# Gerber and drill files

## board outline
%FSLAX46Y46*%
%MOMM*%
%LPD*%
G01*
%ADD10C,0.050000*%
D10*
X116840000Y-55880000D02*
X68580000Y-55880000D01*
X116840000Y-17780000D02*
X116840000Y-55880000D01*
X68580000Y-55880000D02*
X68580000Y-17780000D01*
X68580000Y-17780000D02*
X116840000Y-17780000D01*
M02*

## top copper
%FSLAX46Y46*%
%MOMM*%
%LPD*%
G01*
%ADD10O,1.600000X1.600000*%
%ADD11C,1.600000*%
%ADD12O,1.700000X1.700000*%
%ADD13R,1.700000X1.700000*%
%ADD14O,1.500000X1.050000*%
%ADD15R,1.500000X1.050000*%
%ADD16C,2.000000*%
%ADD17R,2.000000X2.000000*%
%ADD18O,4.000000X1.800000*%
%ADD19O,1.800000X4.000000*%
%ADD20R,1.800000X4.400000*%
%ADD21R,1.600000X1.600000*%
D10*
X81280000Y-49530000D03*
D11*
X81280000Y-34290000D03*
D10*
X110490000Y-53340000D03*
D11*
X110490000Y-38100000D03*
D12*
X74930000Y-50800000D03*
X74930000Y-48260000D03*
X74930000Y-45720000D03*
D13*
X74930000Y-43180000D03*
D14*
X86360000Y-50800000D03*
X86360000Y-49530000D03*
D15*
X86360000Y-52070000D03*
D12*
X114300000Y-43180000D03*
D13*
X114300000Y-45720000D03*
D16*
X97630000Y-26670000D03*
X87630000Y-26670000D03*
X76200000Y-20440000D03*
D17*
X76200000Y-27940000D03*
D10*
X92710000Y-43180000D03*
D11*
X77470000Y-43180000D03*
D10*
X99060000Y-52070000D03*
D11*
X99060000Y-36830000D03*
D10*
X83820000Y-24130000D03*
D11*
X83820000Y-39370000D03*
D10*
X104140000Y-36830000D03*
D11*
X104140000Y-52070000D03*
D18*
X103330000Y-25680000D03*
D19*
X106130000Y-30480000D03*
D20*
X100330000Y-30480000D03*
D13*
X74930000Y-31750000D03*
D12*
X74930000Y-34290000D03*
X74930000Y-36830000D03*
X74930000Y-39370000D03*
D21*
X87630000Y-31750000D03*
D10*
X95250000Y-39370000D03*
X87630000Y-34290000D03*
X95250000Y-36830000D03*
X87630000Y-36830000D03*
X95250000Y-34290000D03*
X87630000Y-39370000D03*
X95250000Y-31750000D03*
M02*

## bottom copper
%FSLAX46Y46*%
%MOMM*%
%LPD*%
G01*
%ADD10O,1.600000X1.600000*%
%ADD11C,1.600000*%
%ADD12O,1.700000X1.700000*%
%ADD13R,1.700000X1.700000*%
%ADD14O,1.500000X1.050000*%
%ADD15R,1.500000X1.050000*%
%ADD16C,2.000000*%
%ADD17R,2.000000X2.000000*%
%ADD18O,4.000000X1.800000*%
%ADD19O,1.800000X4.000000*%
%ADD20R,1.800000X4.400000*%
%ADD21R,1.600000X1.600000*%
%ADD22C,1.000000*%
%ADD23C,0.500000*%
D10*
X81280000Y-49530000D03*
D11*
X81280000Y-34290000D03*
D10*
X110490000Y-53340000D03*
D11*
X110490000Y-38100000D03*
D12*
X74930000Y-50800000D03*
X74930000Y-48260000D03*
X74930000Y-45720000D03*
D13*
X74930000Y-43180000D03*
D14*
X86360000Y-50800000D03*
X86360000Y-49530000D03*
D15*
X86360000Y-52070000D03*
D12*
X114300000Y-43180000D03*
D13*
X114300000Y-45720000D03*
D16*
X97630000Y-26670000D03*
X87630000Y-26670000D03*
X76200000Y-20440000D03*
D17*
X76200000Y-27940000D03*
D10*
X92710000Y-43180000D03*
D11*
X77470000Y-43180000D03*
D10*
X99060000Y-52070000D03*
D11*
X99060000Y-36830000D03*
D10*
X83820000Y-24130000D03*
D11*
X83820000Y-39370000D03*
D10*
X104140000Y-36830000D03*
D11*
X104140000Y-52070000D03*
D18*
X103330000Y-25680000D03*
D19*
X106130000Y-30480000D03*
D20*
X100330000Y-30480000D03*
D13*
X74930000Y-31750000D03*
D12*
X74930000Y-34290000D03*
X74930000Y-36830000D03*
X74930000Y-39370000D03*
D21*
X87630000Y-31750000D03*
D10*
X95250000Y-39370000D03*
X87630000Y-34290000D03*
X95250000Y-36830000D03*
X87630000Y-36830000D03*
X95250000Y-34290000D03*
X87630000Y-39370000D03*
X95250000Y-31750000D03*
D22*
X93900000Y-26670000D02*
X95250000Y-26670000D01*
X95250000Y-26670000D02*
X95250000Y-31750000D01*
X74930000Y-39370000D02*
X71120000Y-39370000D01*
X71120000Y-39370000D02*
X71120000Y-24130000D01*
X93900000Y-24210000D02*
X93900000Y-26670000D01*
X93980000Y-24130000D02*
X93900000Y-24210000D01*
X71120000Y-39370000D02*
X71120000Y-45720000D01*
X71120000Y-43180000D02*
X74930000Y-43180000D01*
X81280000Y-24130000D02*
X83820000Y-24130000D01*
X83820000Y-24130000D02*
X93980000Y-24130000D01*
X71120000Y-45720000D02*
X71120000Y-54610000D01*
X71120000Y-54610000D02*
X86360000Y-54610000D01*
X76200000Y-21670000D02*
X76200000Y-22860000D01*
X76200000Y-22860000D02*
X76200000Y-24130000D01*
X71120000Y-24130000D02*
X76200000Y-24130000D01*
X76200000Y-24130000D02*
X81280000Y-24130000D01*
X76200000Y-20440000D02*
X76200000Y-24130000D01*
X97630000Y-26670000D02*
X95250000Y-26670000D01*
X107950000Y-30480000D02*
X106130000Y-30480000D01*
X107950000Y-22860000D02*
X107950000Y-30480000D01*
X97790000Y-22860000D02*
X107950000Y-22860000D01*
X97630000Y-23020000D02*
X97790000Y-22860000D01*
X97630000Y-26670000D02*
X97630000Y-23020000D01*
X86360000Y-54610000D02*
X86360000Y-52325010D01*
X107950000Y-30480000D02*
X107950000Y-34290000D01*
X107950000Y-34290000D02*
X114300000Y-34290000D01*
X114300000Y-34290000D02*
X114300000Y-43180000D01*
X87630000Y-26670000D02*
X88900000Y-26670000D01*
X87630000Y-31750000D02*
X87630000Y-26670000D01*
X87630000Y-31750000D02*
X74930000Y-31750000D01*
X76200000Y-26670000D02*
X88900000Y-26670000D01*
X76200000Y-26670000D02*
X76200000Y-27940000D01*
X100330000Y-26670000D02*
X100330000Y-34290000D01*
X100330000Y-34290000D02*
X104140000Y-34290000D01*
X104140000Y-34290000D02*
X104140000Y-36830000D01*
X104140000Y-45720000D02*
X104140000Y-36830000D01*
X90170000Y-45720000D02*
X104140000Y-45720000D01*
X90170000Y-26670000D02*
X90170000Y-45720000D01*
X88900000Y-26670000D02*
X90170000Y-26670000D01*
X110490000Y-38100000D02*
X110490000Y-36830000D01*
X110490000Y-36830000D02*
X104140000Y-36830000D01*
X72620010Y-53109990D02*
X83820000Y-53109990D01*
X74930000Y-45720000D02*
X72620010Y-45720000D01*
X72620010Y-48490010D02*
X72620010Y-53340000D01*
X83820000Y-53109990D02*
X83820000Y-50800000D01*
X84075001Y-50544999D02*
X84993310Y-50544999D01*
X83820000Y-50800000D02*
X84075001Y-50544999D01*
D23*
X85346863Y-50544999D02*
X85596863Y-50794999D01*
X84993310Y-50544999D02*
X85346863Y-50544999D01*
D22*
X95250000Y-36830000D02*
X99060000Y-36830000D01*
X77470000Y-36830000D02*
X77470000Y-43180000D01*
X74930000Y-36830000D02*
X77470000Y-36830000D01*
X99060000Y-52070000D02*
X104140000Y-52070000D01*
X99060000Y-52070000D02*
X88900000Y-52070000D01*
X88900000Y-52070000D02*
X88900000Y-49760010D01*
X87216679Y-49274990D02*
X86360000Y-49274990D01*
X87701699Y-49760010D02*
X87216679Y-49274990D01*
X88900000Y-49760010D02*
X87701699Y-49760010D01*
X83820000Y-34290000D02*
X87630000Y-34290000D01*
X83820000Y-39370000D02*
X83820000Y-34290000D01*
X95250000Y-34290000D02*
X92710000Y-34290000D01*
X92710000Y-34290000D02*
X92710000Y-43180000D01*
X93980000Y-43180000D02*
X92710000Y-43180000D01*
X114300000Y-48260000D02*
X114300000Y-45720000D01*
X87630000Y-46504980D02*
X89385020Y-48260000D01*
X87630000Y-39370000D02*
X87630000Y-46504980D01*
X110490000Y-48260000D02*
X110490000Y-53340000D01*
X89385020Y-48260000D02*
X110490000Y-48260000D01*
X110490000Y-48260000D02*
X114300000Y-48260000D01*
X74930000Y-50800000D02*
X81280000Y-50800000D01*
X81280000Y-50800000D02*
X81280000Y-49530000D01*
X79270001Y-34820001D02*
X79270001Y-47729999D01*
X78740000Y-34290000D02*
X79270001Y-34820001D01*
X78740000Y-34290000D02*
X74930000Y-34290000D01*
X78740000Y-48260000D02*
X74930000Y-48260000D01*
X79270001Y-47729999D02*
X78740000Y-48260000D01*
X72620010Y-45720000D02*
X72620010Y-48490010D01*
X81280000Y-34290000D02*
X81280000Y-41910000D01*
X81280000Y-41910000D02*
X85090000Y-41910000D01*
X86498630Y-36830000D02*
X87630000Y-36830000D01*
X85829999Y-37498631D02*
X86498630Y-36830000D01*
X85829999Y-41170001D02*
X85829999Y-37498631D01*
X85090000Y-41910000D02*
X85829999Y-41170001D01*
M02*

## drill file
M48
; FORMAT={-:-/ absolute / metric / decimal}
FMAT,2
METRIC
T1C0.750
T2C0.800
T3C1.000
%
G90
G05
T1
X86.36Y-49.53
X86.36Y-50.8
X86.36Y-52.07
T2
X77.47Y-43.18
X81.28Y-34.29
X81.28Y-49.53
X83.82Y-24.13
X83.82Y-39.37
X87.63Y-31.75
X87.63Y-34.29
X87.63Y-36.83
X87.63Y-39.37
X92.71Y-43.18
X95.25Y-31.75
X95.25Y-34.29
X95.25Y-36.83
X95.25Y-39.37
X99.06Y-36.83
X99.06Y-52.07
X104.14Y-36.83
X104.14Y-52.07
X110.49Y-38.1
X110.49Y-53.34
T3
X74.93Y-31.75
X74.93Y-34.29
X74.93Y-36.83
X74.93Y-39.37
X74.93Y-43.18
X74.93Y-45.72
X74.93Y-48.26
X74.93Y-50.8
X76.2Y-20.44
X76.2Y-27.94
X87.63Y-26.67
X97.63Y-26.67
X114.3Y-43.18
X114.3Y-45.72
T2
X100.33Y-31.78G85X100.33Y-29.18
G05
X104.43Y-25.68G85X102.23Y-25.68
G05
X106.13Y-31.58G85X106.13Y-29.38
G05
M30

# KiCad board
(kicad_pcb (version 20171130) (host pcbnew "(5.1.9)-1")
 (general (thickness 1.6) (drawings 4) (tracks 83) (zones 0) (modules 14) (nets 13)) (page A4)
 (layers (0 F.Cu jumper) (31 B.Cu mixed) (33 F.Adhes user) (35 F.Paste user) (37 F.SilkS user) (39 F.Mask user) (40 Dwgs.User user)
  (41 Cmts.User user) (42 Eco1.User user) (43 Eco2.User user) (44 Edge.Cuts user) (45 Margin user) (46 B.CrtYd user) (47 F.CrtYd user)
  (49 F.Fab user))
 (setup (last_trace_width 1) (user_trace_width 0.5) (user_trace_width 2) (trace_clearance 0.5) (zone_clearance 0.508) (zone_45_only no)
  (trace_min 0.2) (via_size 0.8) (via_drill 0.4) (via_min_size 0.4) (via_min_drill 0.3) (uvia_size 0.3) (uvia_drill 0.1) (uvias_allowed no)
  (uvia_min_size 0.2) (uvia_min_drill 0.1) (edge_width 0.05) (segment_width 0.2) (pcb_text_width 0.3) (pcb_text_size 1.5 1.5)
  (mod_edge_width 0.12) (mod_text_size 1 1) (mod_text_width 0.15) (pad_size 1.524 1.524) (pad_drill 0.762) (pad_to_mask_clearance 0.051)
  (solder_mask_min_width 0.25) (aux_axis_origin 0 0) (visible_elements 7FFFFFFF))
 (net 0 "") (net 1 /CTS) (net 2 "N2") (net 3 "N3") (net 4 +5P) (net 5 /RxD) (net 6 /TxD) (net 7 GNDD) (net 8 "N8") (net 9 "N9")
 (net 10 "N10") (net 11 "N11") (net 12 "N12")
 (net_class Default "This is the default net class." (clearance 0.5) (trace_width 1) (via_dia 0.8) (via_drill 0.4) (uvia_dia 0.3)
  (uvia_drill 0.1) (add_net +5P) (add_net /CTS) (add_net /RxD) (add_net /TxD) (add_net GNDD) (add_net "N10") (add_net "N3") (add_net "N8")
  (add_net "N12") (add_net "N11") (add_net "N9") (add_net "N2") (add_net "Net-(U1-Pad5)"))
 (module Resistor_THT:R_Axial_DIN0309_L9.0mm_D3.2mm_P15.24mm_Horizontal (layer F.Cu) (at 81.28 34.29 270)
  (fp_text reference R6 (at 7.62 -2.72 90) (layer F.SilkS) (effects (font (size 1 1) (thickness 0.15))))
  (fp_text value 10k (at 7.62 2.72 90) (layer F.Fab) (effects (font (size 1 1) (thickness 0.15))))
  (pad 2 thru_hole oval (at 15.24 0 270) (size 1.6 1.6) (drill 0.8) (layers *.Cu *.Mask) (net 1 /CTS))
  (pad 1 thru_hole circle (at 0 0 270) (size 1.6 1.6) (drill 0.8) (layers *.Cu *.Mask) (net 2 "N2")))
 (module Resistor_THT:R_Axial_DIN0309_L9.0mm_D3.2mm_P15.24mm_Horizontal (layer F.Cu) (at 110.49 38.1 270)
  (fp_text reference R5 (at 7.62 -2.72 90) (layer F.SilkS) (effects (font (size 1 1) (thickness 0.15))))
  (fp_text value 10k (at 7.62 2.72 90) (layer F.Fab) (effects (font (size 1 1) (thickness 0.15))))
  (pad 2 thru_hole oval (at 15.24 0 270) (size 1.6 1.6) (drill 0.8) (layers *.Cu *.Mask) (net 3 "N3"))
  (pad 1 thru_hole circle (at 0 0 270) (size 1.6 1.6) (drill 0.8) (layers *.Cu *.Mask) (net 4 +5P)))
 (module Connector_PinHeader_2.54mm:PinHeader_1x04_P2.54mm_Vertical (layer F.Cu) (at 74.93 43.18)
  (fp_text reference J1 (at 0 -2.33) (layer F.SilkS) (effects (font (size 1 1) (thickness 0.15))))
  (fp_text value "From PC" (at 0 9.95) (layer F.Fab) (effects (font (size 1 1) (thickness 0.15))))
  (pad 4 thru_hole oval (at 0 7.62) (size 1.7 1.7) (drill 1) (layers *.Cu *.Mask) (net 1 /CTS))
  (pad 3 thru_hole oval (at 0 5.08) (size 1.7 1.7) (drill 1) (layers *.Cu *.Mask) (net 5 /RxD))
  (pad 2 thru_hole oval (at 0 2.54) (size 1.7 1.7) (drill 1) (layers *.Cu *.Mask) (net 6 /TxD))
  (pad 1 thru_hole rect (at 0 0) (size 1.7 1.7) (drill 1) (layers *.Cu *.Mask) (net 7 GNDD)))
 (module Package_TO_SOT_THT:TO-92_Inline (layer F.Cu) (at 86.36 52.07 90)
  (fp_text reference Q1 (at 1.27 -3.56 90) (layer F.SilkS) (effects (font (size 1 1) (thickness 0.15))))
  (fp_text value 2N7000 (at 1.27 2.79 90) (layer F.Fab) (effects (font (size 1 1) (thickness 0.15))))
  (pad 2 thru_hole oval (at 1.27 0 90) (size 1.05 1.5) (drill 0.75) (layers *.Cu *.Mask) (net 6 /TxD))
  (pad 3 thru_hole oval (at 2.54 0 90) (size 1.05 1.5) (drill 0.75) (layers *.Cu *.Mask) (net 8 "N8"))
  (pad 1 thru_hole rect (at 0 0 90) (size 1.05 1.5) (drill 0.75) (layers *.Cu *.Mask) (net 7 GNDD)))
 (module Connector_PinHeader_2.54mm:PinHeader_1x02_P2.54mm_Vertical (layer F.Cu) (at 114.3 45.72 180)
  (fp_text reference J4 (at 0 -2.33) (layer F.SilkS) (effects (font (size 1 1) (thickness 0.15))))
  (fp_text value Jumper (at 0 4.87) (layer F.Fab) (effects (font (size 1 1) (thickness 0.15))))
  (pad 2 thru_hole oval (at 0 2.54 180) (size 1.7 1.7) (drill 1) (layers *.Cu *.Mask) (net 7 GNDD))
  (pad 1 thru_hole rect (at 0 0 180) (size 1.7 1.7) (drill 1) (layers *.Cu *.Mask) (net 3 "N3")))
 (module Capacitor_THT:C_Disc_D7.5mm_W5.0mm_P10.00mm (layer F.Cu) (at 87.63 26.67)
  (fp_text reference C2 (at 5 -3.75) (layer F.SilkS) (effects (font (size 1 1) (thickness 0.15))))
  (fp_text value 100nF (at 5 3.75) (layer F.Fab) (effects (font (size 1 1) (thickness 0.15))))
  (pad 2 thru_hole circle (at 10 0) (size 2 2) (drill 1) (layers *.Cu *.Mask) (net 7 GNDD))
  (pad 1 thru_hole circle (at 0 0) (size 2 2) (drill 1) (layers *.Cu *.Mask) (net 4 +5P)))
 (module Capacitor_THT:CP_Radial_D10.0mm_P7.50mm (layer F.Cu) (at 76.2 27.94 90)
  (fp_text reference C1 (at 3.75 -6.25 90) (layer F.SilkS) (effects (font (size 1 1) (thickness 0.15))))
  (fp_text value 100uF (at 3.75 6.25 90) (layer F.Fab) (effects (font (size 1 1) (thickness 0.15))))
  (pad 2 thru_hole circle (at 7.5 0 90) (size 2 2) (drill 1) (layers *.Cu *.Mask) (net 7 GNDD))
  (pad 1 thru_hole rect (at 0 0 90) (size 2 2) (drill 1) (layers *.Cu *.Mask) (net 4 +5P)))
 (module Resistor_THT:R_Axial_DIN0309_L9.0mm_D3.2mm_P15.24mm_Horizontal (layer F.Cu) (at 77.47 43.18)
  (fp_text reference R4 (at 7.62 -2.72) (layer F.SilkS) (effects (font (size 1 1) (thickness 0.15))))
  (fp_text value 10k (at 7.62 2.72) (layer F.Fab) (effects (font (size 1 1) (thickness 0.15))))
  (pad 2 thru_hole oval (at 15.24 0) (size 1.6 1.6) (drill 0.8) (layers *.Cu *.Mask) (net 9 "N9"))
  (pad 1 thru_hole circle (at 0 0) (size 1.6 1.6) (drill 0.8) (layers *.Cu *.Mask) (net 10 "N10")))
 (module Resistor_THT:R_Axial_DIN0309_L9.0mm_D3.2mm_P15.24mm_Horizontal (layer F.Cu) (at 99.06 36.83 270)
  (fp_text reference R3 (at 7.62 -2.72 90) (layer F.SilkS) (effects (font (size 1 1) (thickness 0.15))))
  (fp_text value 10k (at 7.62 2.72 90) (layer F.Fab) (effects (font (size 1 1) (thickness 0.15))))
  (pad 2 thru_hole oval (at 15.24 0 270) (size 1.6 1.6) (drill 0.8) (layers *.Cu *.Mask) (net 8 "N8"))
  (pad 1 thru_hole circle (at 0 0 270) (size 1.6 1.6) (drill 0.8) (layers *.Cu *.Mask) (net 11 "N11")))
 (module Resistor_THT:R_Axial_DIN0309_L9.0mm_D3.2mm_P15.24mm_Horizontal (layer F.Cu) (at 83.82 39.37 90)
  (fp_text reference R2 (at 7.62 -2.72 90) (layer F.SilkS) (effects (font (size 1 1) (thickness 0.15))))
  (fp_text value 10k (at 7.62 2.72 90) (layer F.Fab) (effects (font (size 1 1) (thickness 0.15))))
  (pad 2 thru_hole oval (at 15.24 0 90) (size 1.6 1.6) (drill 0.8) (layers *.Cu *.Mask) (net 7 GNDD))
  (pad 1 thru_hole circle (at 0 0 90) (size 1.6 1.6) (drill 0.8) (layers *.Cu *.Mask) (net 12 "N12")))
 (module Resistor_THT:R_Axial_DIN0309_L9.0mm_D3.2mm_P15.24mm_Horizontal (layer F.Cu) (at 104.14 52.07 90)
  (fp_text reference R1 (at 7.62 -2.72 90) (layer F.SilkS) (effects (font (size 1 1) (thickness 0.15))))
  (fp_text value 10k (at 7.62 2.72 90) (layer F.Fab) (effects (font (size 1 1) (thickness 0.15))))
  (pad 2 thru_hole oval (at 15.24 0 90) (size 1.6 1.6) (drill 0.8) (layers *.Cu *.Mask) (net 4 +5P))
  (pad 1 thru_hole circle (at 0 0 90) (size 1.6 1.6) (drill 0.8) (layers *.Cu *.Mask) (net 8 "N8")))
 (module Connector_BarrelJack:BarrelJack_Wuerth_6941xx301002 (layer F.Cu) (at 100.33 30.48 90)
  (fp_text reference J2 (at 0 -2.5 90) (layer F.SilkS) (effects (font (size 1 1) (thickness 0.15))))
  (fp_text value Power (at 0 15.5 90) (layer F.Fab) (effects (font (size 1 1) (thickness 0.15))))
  (pad 3 thru_hole oval (at 4.8 3 180) (size 4 1.8) (drill oval 3 0.8) (layers *.Cu *.Mask))
  (pad 2 thru_hole oval (at 0 5.8 90) (size 4 1.8) (drill oval 3 0.8) (layers *.Cu *.Mask) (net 7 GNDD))
  (pad 1 thru_hole rect (at 0 0 90) (size 4.4 1.8) (drill oval 3.4 0.8) (layers *.Cu *.Mask) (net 4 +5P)))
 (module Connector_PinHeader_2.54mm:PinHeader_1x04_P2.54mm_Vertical (layer F.Cu) (at 74.93 31.75)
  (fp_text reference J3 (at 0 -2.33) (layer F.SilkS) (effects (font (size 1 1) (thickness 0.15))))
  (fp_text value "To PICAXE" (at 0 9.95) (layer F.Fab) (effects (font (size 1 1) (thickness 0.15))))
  (pad 1 thru_hole rect (at 0 0) (size 1.7 1.7) (drill 1) (layers *.Cu *.Mask) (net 4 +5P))
  (pad 2 thru_hole oval (at 0 2.54) (size 1.7 1.7) (drill 1) (layers *.Cu *.Mask) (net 5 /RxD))
  (pad 3 thru_hole oval (at 0 5.08) (size 1.7 1.7) (drill 1) (layers *.Cu *.Mask) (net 10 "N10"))
  (pad 4 thru_hole oval (at 0 7.62) (size 1.7 1.7) (drill 1) (layers *.Cu *.Mask) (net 7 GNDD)))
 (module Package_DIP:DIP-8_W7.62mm (layer F.Cu) (at 87.63 31.75)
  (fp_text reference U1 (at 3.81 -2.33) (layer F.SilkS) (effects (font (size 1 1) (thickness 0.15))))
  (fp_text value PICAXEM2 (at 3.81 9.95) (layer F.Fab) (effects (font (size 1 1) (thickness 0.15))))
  (pad 1 thru_hole rect (at 0 0) (size 1.6 1.6) (drill 0.8) (layers *.Cu *.Mask) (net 4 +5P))
  (pad 5 thru_hole oval (at 7.62 7.62) (size 1.6 1.6) (drill 0.8) (layers *.Cu *.Mask))
  (pad 2 thru_hole oval (at 0 2.54) (size 1.6 1.6) (drill 0.8) (layers *.Cu *.Mask) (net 12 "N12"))
  (pad 6 thru_hole oval (at 7.62 5.08) (size 1.6 1.6) (drill 0.8) (layers *.Cu *.Mask) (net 11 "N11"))
  (pad 3 thru_hole oval (at 0 5.08) (size 1.6 1.6) (drill 0.8) (layers *.Cu *.Mask) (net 2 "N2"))
  (pad 7 thru_hole oval (at 7.62 2.54) (size 1.6 1.6) (drill 0.8) (layers *.Cu *.Mask) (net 9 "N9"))
  (pad 4 thru_hole oval (at 0 7.62) (size 1.6 1.6) (drill 0.8) (layers *.Cu *.Mask) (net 3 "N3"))
  (pad 8 thru_hole oval (at 7.62 0) (size 1.6 1.6) (drill 0.8) (layers *.Cu *.Mask) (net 7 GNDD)))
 (gr_line (start 116.84 55.88) (end 68.58 55.88) (layer Edge.Cuts) (width 0.05))
 (gr_line (start 116.84 17.78) (end 116.84 55.88) (layer Edge.Cuts) (width 0.05))
 (gr_line (start 68.58 55.88) (end 68.58 17.78) (layer Edge.Cuts) (width 0.05))
 (gr_line (start 68.58 17.78) (end 116.84 17.78) (layer Edge.Cuts) (width 0.05))
 (segment (start 93.9 26.67) (end 95.25 26.67) (width 1) (layer B.Cu) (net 7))
 (segment (start 95.25 26.67) (end 95.25 31.75) (width 1) (layer B.Cu) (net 7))
 (segment (start 74.93 39.37) (end 71.12 39.37) (width 1) (layer B.Cu) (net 7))
 (segment (start 71.12 39.37) (end 71.12 24.13) (width 1) (layer B.Cu) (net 7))
 (segment (start 93.9 24.21) (end 93.9 26.67) (width 1) (layer B.Cu) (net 7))
 (segment (start 93.98 24.13) (end 93.9 24.21) (width 1) (layer B.Cu) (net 7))
 (segment (start 71.12 39.37) (end 71.12 45.72) (width 1) (layer B.Cu) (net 7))
 (segment (start 71.12 43.18) (end 74.93 43.18) (width 1) (layer B.Cu) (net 7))
 (segment (start 81.28 24.13) (end 83.82 24.13) (width 1) (layer B.Cu) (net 7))
 (segment (start 83.82 24.13) (end 93.98 24.13) (width 1) (layer B.Cu) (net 7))
 (segment (start 71.12 45.72) (end 71.12 54.61) (width 1) (layer B.Cu) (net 7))
 (segment (start 71.12 54.61) (end 86.36 54.61) (width 1) (layer B.Cu) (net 7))
 (segment (start 76.2 21.67) (end 76.2 22.86) (width 1) (layer B.Cu) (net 7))
 (segment (start 76.2 22.86) (end 76.2 24.13) (width 1) (layer B.Cu) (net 7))
 (segment (start 71.12 24.13) (end 76.2 24.13) (width 1) (layer B.Cu) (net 7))
 (segment (start 76.2 24.13) (end 81.28 24.13) (width 1) (layer B.Cu) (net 7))
 (segment (start 76.2 20.44) (end 76.2 24.13) (width 1) (layer B.Cu) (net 7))
 (segment (start 97.63 26.67) (end 95.25 26.67) (width 1) (layer B.Cu) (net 7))
 (segment (start 107.95 30.48) (end 106.13 30.48) (width 1) (layer B.Cu) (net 7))
 (segment (start 107.95 22.86) (end 107.95 30.48) (width 1) (layer B.Cu) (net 7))
 (segment (start 97.79 22.86) (end 107.95 22.86) (width 1) (layer B.Cu) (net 7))
 (segment (start 97.63 23.02) (end 97.79 22.86) (width 1) (layer B.Cu) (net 7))
 (segment (start 97.63 26.67) (end 97.63 23.02) (width 1) (layer B.Cu) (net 7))
 (segment (start 86.36 54.61) (end 86.36 52.32501) (width 1) (layer B.Cu) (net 7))
 (segment (start 107.95 30.48) (end 107.95 34.29) (width 1) (layer B.Cu) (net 7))
 (segment (start 107.95 34.29) (end 114.3 34.29) (width 1) (layer B.Cu) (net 7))
 (segment (start 114.3 34.29) (end 114.3 43.18) (width 1) (layer B.Cu) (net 7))
 (segment (start 87.63 26.67) (end 88.9 26.67) (width 1) (layer B.Cu) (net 4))
 (segment (start 87.63 31.75) (end 87.63 26.67) (width 1) (layer B.Cu) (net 4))
 (segment (start 87.63 31.75) (end 74.93 31.75) (width 1) (layer B.Cu) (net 4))
 (segment (start 76.2 26.67) (end 88.9 26.67) (width 1) (layer B.Cu) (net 4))
 (segment (start 76.2 26.67) (end 76.2 27.94) (width 1) (layer B.Cu) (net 4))
 (segment (start 100.33 26.67) (end 100.33 34.29) (width 1) (layer B.Cu) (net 4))
 (segment (start 100.33 34.29) (end 104.14 34.29) (width 1) (layer B.Cu) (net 4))
 (segment (start 104.14 34.29) (end 104.14 36.83) (width 1) (layer B.Cu) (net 4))
 (segment (start 104.14 45.72) (end 104.14 36.83) (width 1) (layer B.Cu) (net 4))
 (segment (start 90.17 45.72) (end 104.14 45.72) (width 1) (layer B.Cu) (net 4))
 (segment (start 90.17 26.67) (end 90.17 45.72) (width 1) (layer B.Cu) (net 4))
 (segment (start 88.9 26.67) (end 90.17 26.67) (width 1) (layer B.Cu) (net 4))
 (segment (start 110.49 38.1) (end 110.49 36.83) (width 1) (layer B.Cu) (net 4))
 (segment (start 110.49 36.83) (end 104.14 36.83) (width 1) (layer B.Cu) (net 4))
 (segment (start 72.62001 53.10999) (end 83.82 53.10999) (width 1) (layer B.Cu) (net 6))
 (segment (start 74.93 45.72) (end 72.62001 45.72) (width 1) (layer B.Cu) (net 6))
 (segment (start 72.62001 48.49001) (end 72.62001 53.34) (width 1) (layer B.Cu) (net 6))
 (segment (start 83.82 53.10999) (end 83.82 50.8) (width 1) (layer B.Cu) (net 6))
 (segment (start 84.075001 50.544999) (end 84.99331 50.544999) (width 1) (layer B.Cu) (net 6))
 (segment (start 83.82 50.8) (end 84.075001 50.544999) (width 1) (layer B.Cu) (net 6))
 (segment (start 85.346863 50.544999) (end 85.596863 50.794999) (width 0.5) (layer B.Cu) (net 6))
 (segment (start 84.99331 50.544999) (end 85.346863 50.544999) (width 0.5) (layer B.Cu) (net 6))
 (segment (start 95.25 36.83) (end 99.06 36.83) (width 1) (layer B.Cu) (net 11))
 (segment (start 77.47 36.83) (end 77.47 43.18) (width 1) (layer B.Cu) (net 10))
 (segment (start 74.93 36.83) (end 77.47 36.83) (width 1) (layer B.Cu) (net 10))
 (segment (start 99.06 52.07) (end 104.14 52.07) (width 1) (layer B.Cu) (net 8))
 (segment (start 99.06 52.07) (end 88.9 52.07) (width 1) (layer B.Cu) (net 8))
 (segment (start 88.9 52.07) (end 88.9 49.76001) (width 1) (layer B.Cu) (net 8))
 (segment (start 87.216679 49.27499) (end 86.36 49.27499) (width 1) (layer B.Cu) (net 8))
 (segment (start 87.701699 49.76001) (end 87.216679 49.27499) (width 1) (layer B.Cu) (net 8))
 (segment (start 88.9 49.76001) (end 87.701699 49.76001) (width 1) (layer B.Cu) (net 8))
 (segment (start 83.82 34.29) (end 87.63 34.29) (width 1) (layer B.Cu) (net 12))
 (segment (start 83.82 39.37) (end 83.82 34.29) (width 1) (layer B.Cu) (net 12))
 (segment (start 95.25 34.29) (end 92.71 34.29) (width 1) (layer B.Cu) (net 9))
 (segment (start 92.71 34.29) (end 92.71 43.18) (width 1) (layer B.Cu) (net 9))
 (segment (start 93.98 43.18) (end 92.71 43.18) (width 1) (layer B.Cu) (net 9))
 (segment (start 114.3 48.26) (end 114.3 45.72) (width 1) (layer B.Cu) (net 3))
 (segment (start 87.63 46.50498) (end 89.38502 48.26) (width 1) (layer B.Cu) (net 3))
 (segment (start 87.63 39.37) (end 87.63 46.50498) (width 1) (layer B.Cu) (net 3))
 (segment (start 110.49 48.26) (end 110.49 53.34) (width 1) (layer B.Cu) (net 3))
 (segment (start 89.38502 48.26) (end 110.49 48.26) (width 1) (layer B.Cu) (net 3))
 (segment (start 110.49 48.26) (end 114.3 48.26) (width 1) (layer B.Cu) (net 3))
 (segment (start 74.93 50.8) (end 81.28 50.8) (width 1) (layer B.Cu) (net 1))
 (segment (start 81.28 50.8) (end 81.28 49.53) (width 1) (layer B.Cu) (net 1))
 (segment (start 79.270001 34.820001) (end 79.270001 47.729999) (width 1) (layer B.Cu) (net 5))
 (segment (start 78.74 34.29) (end 79.270001 34.820001) (width 1) (layer B.Cu) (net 5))
 (segment (start 78.74 34.29) (end 74.93 34.29) (width 1) (layer B.Cu) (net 5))
 (segment (start 78.74 48.26) (end 74.93 48.26) (width 1) (layer B.Cu) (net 5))
 (segment (start 79.270001 47.729999) (end 78.74 48.26) (width 1) (layer B.Cu) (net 5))
 (segment (start 72.62001 45.72) (end 72.62001 48.49001) (width 1) (layer B.Cu) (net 6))
 (segment (start 81.28 34.29) (end 81.28 41.91) (width 1) (layer B.Cu) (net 2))
 (segment (start 81.28 41.91) (end 85.09 41.91) (width 1) (layer B.Cu) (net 2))
 (segment (start 86.49863 36.83) (end 87.63 36.83) (width 1) (layer B.Cu) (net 2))
 (segment (start 85.829999 37.498631) (end 86.49863 36.83) (width 1) (layer B.Cu) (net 2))
 (segment (start 85.829999 41.170001) (end 85.829999 37.498631) (width 1) (layer B.Cu) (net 2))
 (segment (start 85.09 41.91) (end 85.829999 41.170001) (width 1) (layer B.Cu) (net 2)))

